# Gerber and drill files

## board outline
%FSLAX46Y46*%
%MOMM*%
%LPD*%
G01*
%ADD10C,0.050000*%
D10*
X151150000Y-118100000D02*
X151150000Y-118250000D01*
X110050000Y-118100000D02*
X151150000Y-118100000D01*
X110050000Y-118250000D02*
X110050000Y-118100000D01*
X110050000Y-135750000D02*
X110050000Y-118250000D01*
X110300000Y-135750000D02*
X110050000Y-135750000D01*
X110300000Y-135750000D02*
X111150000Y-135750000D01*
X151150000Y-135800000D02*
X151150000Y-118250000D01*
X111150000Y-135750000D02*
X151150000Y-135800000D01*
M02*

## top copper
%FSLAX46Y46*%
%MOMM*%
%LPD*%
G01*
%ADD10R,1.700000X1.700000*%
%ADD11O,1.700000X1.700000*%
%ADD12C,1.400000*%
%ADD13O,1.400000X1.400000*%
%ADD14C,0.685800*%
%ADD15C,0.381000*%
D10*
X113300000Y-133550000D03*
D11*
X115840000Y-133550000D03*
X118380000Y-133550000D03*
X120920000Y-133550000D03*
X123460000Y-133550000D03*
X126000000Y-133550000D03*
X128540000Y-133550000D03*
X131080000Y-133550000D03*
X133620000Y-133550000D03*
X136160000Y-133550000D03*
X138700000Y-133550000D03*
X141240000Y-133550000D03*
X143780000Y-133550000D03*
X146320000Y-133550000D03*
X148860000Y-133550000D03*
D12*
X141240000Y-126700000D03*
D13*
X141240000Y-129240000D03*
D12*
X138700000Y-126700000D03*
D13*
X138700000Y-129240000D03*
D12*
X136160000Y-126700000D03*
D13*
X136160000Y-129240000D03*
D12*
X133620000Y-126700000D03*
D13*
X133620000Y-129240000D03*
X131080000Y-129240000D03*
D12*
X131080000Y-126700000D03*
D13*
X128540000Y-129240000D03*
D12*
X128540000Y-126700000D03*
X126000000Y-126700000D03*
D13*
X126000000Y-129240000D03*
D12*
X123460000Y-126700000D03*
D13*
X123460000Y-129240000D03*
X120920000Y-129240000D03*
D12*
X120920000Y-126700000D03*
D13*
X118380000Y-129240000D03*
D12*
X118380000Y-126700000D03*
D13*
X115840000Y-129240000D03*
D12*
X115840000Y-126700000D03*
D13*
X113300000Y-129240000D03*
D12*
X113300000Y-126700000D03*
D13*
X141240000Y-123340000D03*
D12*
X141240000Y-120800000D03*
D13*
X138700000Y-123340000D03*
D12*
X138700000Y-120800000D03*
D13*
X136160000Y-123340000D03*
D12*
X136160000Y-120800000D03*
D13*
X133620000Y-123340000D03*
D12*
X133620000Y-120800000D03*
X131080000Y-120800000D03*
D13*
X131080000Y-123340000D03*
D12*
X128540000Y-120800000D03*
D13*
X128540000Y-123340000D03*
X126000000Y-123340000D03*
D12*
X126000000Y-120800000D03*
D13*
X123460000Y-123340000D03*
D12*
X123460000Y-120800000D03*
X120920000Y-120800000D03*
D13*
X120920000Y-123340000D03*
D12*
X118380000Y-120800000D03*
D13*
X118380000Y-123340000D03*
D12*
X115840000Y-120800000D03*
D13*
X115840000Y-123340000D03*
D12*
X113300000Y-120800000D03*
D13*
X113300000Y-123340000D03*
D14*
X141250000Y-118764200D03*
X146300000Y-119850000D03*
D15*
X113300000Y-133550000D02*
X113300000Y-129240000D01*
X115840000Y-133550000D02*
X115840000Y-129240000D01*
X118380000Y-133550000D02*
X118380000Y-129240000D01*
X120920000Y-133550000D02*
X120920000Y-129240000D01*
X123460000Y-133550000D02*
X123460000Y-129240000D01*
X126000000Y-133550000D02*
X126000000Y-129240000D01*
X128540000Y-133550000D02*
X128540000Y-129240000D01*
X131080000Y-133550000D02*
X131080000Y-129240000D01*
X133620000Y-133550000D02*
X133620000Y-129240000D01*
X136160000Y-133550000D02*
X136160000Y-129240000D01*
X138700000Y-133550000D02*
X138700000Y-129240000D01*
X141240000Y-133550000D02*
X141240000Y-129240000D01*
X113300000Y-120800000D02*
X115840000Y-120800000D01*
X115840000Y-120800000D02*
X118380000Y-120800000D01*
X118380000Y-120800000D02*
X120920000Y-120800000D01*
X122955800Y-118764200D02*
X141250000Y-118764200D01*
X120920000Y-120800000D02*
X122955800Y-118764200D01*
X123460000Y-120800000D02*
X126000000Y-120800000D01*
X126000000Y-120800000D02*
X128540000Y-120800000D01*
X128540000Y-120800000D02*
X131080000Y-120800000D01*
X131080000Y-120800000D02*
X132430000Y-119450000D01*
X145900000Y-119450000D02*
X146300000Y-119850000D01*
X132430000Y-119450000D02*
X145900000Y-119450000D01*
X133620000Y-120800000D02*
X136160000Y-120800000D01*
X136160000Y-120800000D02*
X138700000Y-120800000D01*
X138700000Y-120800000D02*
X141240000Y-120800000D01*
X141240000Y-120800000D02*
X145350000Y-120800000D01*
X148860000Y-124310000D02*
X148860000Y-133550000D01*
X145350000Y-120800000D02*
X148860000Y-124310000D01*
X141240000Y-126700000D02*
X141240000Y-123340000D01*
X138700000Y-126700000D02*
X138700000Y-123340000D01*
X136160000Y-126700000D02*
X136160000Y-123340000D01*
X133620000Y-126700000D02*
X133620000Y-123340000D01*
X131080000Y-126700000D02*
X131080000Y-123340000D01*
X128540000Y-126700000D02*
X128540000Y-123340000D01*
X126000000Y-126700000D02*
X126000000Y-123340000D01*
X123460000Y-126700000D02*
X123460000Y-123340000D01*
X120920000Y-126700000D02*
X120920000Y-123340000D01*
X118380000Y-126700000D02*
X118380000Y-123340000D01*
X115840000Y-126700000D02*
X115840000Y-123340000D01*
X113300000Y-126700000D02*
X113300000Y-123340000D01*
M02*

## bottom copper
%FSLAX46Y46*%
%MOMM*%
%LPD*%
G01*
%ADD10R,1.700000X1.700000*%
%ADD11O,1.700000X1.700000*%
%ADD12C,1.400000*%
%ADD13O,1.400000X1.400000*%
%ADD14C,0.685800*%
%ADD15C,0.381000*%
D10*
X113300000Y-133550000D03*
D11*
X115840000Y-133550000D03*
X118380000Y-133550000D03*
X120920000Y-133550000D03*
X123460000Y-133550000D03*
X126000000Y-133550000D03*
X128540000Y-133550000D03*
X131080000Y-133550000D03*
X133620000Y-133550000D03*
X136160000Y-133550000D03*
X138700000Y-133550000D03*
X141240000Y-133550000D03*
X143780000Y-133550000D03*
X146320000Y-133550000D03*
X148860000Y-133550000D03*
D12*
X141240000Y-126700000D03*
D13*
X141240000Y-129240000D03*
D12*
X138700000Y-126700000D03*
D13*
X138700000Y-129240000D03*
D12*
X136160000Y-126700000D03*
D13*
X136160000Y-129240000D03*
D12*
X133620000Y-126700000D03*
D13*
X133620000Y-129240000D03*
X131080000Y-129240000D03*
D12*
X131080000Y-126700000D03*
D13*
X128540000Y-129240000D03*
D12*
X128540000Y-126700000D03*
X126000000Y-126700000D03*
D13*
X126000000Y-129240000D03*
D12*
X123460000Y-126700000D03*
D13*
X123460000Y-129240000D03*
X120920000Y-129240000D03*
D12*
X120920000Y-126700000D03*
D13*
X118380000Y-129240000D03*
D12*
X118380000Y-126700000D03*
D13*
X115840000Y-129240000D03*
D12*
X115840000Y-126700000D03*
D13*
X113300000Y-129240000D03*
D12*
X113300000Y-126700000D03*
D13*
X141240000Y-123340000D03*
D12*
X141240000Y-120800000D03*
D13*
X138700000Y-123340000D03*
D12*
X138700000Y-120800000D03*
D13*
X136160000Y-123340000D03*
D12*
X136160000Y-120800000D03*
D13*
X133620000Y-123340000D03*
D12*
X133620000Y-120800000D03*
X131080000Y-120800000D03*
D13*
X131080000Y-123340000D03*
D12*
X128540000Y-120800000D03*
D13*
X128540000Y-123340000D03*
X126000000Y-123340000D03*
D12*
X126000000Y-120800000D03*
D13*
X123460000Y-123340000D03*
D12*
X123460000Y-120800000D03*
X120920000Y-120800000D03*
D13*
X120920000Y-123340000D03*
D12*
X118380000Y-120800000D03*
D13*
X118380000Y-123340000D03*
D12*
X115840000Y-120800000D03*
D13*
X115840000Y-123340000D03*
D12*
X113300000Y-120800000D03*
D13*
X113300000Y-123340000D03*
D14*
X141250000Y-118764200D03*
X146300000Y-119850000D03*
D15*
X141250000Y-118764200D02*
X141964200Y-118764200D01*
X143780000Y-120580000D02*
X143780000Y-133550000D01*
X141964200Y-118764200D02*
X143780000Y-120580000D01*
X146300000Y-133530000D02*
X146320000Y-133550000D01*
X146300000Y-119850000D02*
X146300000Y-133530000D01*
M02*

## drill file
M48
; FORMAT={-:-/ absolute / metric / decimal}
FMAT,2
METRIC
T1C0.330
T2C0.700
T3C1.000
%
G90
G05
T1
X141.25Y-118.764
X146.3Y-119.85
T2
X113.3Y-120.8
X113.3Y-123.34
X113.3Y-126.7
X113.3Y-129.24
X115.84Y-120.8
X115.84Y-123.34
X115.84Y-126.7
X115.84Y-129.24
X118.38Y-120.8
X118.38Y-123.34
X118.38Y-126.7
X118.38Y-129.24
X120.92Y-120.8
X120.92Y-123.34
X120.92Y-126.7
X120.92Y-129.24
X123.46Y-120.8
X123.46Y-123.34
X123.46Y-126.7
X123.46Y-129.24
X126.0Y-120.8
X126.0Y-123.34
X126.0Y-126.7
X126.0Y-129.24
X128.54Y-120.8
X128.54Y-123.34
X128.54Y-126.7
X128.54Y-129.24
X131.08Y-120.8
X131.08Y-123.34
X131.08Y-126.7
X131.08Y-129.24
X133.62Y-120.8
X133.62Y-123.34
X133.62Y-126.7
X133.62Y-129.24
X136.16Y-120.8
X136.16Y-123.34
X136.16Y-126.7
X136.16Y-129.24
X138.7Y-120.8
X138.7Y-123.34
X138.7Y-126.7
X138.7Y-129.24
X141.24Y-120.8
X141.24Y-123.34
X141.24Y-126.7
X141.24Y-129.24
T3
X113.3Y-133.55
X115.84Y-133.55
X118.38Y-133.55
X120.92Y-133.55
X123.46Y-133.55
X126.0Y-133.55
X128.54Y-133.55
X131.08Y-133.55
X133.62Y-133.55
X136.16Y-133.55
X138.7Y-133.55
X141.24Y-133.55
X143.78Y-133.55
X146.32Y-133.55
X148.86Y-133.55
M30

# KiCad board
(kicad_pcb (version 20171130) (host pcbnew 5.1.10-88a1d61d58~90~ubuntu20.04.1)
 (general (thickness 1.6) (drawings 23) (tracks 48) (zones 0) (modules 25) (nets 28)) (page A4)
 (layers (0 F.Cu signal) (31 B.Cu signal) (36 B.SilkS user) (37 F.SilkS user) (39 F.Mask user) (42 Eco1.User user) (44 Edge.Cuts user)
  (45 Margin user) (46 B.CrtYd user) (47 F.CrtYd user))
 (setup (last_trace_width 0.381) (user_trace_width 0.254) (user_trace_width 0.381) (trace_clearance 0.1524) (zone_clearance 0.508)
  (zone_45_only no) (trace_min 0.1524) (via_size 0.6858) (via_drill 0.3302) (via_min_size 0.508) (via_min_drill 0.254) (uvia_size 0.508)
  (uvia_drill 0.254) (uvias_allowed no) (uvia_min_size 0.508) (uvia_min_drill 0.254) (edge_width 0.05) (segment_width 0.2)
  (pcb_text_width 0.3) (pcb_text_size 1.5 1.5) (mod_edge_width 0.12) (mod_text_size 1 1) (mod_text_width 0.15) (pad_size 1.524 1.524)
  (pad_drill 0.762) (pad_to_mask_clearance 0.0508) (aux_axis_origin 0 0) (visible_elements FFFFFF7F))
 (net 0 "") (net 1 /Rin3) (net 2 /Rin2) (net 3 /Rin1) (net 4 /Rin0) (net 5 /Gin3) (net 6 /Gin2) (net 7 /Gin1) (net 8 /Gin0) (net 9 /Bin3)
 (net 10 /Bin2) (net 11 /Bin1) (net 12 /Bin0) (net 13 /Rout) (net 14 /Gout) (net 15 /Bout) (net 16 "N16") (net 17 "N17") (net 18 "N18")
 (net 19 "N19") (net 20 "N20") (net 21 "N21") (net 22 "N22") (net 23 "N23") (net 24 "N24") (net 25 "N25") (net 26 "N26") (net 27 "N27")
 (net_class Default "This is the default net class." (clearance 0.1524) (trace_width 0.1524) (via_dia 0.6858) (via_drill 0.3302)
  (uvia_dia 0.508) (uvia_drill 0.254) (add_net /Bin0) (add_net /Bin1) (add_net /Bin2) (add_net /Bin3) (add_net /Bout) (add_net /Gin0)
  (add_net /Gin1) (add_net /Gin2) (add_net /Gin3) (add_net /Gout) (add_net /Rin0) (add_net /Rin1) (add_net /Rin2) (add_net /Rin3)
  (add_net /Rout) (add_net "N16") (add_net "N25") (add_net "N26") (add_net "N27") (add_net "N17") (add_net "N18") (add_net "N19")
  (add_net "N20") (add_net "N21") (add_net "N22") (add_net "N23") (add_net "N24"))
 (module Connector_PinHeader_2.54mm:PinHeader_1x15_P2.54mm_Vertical (layer F.Cu) (at 113.3 133.55 90)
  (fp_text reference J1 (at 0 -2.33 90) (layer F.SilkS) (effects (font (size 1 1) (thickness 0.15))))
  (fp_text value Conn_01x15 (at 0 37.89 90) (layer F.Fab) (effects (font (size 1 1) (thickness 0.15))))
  (pad 1 thru_hole rect (at 0 0 90) (size 1.7 1.7) (drill 1) (layers *.Cu *.Mask) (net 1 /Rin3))
  (pad 2 thru_hole oval (at 0 2.54 90) (size 1.7 1.7) (drill 1) (layers *.Cu *.Mask) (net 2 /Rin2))
  (pad 3 thru_hole oval (at 0 5.08 90) (size 1.7 1.7) (drill 1) (layers *.Cu *.Mask) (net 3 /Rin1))
  (pad 4 thru_hole oval (at 0 7.62 90) (size 1.7 1.7) (drill 1) (layers *.Cu *.Mask) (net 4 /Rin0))
  (pad 5 thru_hole oval (at 0 10.16 90) (size 1.7 1.7) (drill 1) (layers *.Cu *.Mask) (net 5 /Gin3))
  (pad 6 thru_hole oval (at 0 12.7 90) (size 1.7 1.7) (drill 1) (layers *.Cu *.Mask) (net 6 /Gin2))
  (pad 7 thru_hole oval (at 0 15.24 90) (size 1.7 1.7) (drill 1) (layers *.Cu *.Mask) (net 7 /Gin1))
  (pad 8 thru_hole oval (at 0 17.78 90) (size 1.7 1.7) (drill 1) (layers *.Cu *.Mask) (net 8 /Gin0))
  (pad 9 thru_hole oval (at 0 20.32 90) (size 1.7 1.7) (drill 1) (layers *.Cu *.Mask) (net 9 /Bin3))
  (pad 10 thru_hole oval (at 0 22.86 90) (size 1.7 1.7) (drill 1) (layers *.Cu *.Mask) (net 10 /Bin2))
  (pad 11 thru_hole oval (at 0 25.4 90) (size 1.7 1.7) (drill 1) (layers *.Cu *.Mask) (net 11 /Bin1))
  (pad 12 thru_hole oval (at 0 27.94 90) (size 1.7 1.7) (drill 1) (layers *.Cu *.Mask) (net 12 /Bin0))
  (pad 13 thru_hole oval (at 0 30.48 90) (size 1.7 1.7) (drill 1) (layers *.Cu *.Mask) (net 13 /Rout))
  (pad 14 thru_hole oval (at 0 33.02 90) (size 1.7 1.7) (drill 1) (layers *.Cu *.Mask) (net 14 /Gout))
  (pad 15 thru_hole oval (at 0 35.56 90) (size 1.7 1.7) (drill 1) (layers *.Cu *.Mask) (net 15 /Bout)))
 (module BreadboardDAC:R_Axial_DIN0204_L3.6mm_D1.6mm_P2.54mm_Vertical (layer F.Cu) (at 141.24 126.7 270)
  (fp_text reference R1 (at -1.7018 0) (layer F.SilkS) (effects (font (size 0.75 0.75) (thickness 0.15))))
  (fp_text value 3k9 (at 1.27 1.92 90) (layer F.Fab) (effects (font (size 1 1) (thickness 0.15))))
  (pad 1 thru_hole circle (at 0 0 270) (size 1.4 1.4) (drill 0.7) (layers *.Cu *.Mask) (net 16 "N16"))
  (pad 2 thru_hole oval (at 2.54 0 270) (size 1.4 1.4) (drill 0.7) (layers *.Cu *.Mask) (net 12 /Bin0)))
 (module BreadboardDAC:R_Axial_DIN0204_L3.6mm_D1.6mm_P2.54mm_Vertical (layer F.Cu) (at 138.7 126.7 270)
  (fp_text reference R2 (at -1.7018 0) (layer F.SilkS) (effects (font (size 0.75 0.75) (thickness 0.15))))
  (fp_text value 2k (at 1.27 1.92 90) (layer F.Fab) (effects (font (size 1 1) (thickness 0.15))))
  (pad 1 thru_hole circle (at 0 0 270) (size 1.4 1.4) (drill 0.7) (layers *.Cu *.Mask) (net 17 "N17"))
  (pad 2 thru_hole oval (at 2.54 0 270) (size 1.4 1.4) (drill 0.7) (layers *.Cu *.Mask) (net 11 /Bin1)))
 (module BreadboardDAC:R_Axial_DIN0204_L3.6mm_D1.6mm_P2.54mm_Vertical (layer F.Cu) (at 136.16 126.7 270)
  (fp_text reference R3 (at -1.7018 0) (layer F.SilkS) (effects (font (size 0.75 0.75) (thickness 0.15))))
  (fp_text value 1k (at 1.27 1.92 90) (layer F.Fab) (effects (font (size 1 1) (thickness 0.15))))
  (pad 1 thru_hole circle (at 0 0 270) (size 1.4 1.4) (drill 0.7) (layers *.Cu *.Mask) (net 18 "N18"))
  (pad 2 thru_hole oval (at 2.54 0 270) (size 1.4 1.4) (drill 0.7) (layers *.Cu *.Mask) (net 10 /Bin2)))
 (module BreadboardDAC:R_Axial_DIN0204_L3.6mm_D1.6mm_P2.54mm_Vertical (layer F.Cu) (at 133.62 126.7 270)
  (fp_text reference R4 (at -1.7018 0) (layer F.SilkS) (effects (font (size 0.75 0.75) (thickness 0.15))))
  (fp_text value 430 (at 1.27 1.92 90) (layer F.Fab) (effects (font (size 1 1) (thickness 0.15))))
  (pad 1 thru_hole circle (at 0 0 270) (size 1.4 1.4) (drill 0.7) (layers *.Cu *.Mask) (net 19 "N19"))
  (pad 2 thru_hole oval (at 2.54 0 270) (size 1.4 1.4) (drill 0.7) (layers *.Cu *.Mask) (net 9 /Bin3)))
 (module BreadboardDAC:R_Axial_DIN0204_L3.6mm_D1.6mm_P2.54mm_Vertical (layer F.Cu) (at 131.08 126.7 270)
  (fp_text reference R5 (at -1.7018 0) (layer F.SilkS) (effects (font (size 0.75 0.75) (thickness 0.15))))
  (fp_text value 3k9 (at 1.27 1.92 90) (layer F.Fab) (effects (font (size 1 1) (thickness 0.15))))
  (pad 2 thru_hole oval (at 2.54 0 270) (size 1.4 1.4) (drill 0.7) (layers *.Cu *.Mask) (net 8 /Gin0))
  (pad 1 thru_hole circle (at 0 0 270) (size 1.4 1.4) (drill 0.7) (layers *.Cu *.Mask) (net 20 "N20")))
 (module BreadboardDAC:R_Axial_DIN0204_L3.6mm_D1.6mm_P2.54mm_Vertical (layer F.Cu) (at 128.54 126.7 270)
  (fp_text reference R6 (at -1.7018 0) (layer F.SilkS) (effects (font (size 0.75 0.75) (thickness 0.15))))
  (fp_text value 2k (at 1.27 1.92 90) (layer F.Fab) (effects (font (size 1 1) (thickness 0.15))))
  (pad 2 thru_hole oval (at 2.54 0 270) (size 1.4 1.4) (drill 0.7) (layers *.Cu *.Mask) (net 7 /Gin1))
  (pad 1 thru_hole circle (at 0 0 270) (size 1.4 1.4) (drill 0.7) (layers *.Cu *.Mask) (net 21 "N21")))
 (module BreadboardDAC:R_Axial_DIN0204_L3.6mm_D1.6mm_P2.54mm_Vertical (layer F.Cu) (at 126 126.7 270)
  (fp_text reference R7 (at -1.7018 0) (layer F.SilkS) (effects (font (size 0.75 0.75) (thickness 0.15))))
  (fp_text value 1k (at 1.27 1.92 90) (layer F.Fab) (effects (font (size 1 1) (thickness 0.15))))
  (pad 1 thru_hole circle (at 0 0 270) (size 1.4 1.4) (drill 0.7) (layers *.Cu *.Mask) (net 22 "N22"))
  (pad 2 thru_hole oval (at 2.54 0 270) (size 1.4 1.4) (drill 0.7) (layers *.Cu *.Mask) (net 6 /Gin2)))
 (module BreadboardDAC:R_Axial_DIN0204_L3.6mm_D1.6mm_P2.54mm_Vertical (layer F.Cu) (at 123.46 126.7 270)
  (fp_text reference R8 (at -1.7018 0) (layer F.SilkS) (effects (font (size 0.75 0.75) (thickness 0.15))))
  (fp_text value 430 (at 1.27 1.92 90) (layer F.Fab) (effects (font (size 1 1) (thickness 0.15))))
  (pad 1 thru_hole circle (at 0 0 270) (size 1.4 1.4) (drill 0.7) (layers *.Cu *.Mask) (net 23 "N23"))
  (pad 2 thru_hole oval (at 2.54 0 270) (size 1.4 1.4) (drill 0.7) (layers *.Cu *.Mask) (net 5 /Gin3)))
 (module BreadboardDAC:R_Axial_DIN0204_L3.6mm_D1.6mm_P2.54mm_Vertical (layer F.Cu) (at 120.92 126.7 270)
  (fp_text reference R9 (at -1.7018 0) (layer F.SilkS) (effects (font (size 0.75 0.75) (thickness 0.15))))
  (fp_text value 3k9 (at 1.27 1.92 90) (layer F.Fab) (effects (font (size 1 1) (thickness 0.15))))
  (pad 2 thru_hole oval (at 2.54 0 270) (size 1.4 1.4) (drill 0.7) (layers *.Cu *.Mask) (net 4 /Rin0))
  (pad 1 thru_hole circle (at 0 0 270) (size 1.4 1.4) (drill 0.7) (layers *.Cu *.Mask) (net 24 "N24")))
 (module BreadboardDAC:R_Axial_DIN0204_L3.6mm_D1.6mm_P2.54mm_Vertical (layer F.Cu) (at 118.38 126.7 270)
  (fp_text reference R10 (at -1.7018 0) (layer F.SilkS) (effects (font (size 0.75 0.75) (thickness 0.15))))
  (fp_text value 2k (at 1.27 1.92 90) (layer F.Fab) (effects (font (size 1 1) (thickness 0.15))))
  (pad 2 thru_hole oval (at 2.54 0 270) (size 1.4 1.4) (drill 0.7) (layers *.Cu *.Mask) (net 3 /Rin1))
  (pad 1 thru_hole circle (at 0 0 270) (size 1.4 1.4) (drill 0.7) (layers *.Cu *.Mask) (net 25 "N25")))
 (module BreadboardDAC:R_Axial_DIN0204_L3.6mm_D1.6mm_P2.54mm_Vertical (layer F.Cu) (at 115.84 126.7 270)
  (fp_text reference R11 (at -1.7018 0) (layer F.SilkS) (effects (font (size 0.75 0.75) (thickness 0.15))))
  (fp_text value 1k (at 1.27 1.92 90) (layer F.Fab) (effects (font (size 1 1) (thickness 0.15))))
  (pad 2 thru_hole oval (at 2.54 0 270) (size 1.4 1.4) (drill 0.7) (layers *.Cu *.Mask) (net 2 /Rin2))
  (pad 1 thru_hole circle (at 0 0 270) (size 1.4 1.4) (drill 0.7) (layers *.Cu *.Mask) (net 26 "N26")))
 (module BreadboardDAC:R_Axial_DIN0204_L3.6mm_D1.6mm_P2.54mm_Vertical (layer F.Cu) (at 113.3 126.7 270)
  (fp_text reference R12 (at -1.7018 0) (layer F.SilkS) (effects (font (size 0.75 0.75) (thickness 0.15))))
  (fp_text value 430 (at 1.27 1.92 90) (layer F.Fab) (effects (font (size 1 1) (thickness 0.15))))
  (pad 2 thru_hole oval (at 2.54 0 270) (size 1.4 1.4) (drill 0.7) (layers *.Cu *.Mask) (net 1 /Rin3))
  (pad 1 thru_hole circle (at 0 0 270) (size 1.4 1.4) (drill 0.7) (layers *.Cu *.Mask) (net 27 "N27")))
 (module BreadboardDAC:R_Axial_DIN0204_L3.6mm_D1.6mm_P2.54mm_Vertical (layer F.Cu) (at 141.24 120.8 270)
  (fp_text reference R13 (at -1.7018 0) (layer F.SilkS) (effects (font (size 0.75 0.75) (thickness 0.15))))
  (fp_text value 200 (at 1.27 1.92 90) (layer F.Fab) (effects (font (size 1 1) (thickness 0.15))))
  (pad 2 thru_hole oval (at 2.54 0 270) (size 1.4 1.4) (drill 0.7) (layers *.Cu *.Mask) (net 16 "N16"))
  (pad 1 thru_hole circle (at 0 0 270) (size 1.4 1.4) (drill 0.7) (layers *.Cu *.Mask) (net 15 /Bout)))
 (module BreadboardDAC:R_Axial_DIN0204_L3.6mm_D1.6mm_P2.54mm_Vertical (layer F.Cu) (at 138.7 120.8 270)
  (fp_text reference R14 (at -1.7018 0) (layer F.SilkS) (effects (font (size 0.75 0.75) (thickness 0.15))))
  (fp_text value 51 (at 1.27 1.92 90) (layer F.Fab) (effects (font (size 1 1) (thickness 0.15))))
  (pad 2 thru_hole oval (at 2.54 0 270) (size 1.4 1.4) (drill 0.7) (layers *.Cu *.Mask) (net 17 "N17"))
  (pad 1 thru_hole circle (at 0 0 270) (size 1.4 1.4) (drill 0.7) (layers *.Cu *.Mask) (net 15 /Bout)))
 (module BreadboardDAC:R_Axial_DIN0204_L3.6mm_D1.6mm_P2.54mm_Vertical (layer F.Cu) (at 136.16 120.8 270)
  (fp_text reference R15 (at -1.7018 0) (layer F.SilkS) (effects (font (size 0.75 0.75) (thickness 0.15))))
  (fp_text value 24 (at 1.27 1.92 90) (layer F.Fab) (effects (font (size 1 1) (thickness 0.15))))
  (pad 2 thru_hole oval (at 2.54 0 270) (size 1.4 1.4) (drill 0.7) (layers *.Cu *.Mask) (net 18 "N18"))
  (pad 1 thru_hole circle (at 0 0 270) (size 1.4 1.4) (drill 0.7) (layers *.Cu *.Mask) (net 15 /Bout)))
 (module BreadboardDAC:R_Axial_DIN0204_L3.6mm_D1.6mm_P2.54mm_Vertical (layer F.Cu) (at 133.62 120.8 270)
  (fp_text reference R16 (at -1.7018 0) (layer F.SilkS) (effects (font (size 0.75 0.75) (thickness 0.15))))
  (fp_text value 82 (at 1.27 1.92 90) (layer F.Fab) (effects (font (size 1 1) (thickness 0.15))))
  (pad 2 thru_hole oval (at 2.54 0 270) (size 1.4 1.4) (drill 0.7) (layers *.Cu *.Mask) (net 19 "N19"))
  (pad 1 thru_hole circle (at 0 0 270) (size 1.4 1.4) (drill 0.7) (layers *.Cu *.Mask) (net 15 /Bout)))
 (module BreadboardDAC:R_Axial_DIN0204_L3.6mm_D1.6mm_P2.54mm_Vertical (layer F.Cu) (at 131.08 120.8 270)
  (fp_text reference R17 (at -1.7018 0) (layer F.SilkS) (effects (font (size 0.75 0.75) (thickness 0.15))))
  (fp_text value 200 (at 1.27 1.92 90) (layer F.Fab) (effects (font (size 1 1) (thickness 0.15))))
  (pad 1 thru_hole circle (at 0 0 270) (size 1.4 1.4) (drill 0.7) (layers *.Cu *.Mask) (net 14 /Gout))
  (pad 2 thru_hole oval (at 2.54 0 270) (size 1.4 1.4) (drill 0.7) (layers *.Cu *.Mask) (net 20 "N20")))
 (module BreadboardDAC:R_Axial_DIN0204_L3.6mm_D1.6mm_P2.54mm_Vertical (layer F.Cu) (at 128.54 120.8 270)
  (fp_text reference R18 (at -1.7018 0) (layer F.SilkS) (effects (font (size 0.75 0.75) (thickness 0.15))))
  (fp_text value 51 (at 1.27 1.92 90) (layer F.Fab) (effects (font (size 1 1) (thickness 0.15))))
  (pad 1 thru_hole circle (at 0 0 270) (size 1.4 1.4) (drill 0.7) (layers *.Cu *.Mask) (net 14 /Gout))
  (pad 2 thru_hole oval (at 2.54 0 270) (size 1.4 1.4) (drill 0.7) (layers *.Cu *.Mask) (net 21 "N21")))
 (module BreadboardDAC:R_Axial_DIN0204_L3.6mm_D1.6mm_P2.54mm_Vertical (layer F.Cu) (at 126 120.8 270)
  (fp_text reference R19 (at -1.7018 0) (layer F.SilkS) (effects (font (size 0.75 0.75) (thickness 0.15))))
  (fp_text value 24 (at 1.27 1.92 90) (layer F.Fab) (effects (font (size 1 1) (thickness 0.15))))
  (pad 2 thru_hole oval (at 2.54 0 270) (size 1.4 1.4) (drill 0.7) (layers *.Cu *.Mask) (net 22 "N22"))
  (pad 1 thru_hole circle (at 0 0 270) (size 1.4 1.4) (drill 0.7) (layers *.Cu *.Mask) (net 14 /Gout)))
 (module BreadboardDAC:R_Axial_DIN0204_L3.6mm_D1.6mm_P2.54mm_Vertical (layer F.Cu) (at 123.46 120.8 270)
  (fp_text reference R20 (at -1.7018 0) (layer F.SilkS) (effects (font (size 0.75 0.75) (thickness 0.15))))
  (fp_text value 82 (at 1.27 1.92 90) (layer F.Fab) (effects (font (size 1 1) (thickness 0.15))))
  (pad 2 thru_hole oval (at 2.54 0 270) (size 1.4 1.4) (drill 0.7) (layers *.Cu *.Mask) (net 23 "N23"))
  (pad 1 thru_hole circle (at 0 0 270) (size 1.4 1.4) (drill 0.7) (layers *.Cu *.Mask) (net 14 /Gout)))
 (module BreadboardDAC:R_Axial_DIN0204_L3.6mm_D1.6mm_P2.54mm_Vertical (layer F.Cu) (at 120.92 120.8 270)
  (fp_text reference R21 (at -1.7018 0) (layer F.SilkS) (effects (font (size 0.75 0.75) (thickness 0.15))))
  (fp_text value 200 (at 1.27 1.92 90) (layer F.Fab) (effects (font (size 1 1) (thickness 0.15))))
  (pad 1 thru_hole circle (at 0 0 270) (size 1.4 1.4) (drill 0.7) (layers *.Cu *.Mask) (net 13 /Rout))
  (pad 2 thru_hole oval (at 2.54 0 270) (size 1.4 1.4) (drill 0.7) (layers *.Cu *.Mask) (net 24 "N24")))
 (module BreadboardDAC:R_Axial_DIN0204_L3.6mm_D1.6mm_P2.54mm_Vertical (layer F.Cu) (at 118.38 120.8 270)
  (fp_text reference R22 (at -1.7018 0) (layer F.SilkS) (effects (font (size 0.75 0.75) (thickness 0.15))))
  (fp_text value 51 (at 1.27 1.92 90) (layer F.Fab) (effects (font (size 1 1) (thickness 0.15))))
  (pad 1 thru_hole circle (at 0 0 270) (size 1.4 1.4) (drill 0.7) (layers *.Cu *.Mask) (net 13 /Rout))
  (pad 2 thru_hole oval (at 2.54 0 270) (size 1.4 1.4) (drill 0.7) (layers *.Cu *.Mask) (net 25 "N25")))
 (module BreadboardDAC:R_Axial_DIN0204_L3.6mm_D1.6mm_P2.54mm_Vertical (layer F.Cu) (at 115.84 120.8 270)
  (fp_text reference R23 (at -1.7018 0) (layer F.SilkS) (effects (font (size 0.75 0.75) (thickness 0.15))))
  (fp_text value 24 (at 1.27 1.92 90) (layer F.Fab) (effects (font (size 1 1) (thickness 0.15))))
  (pad 1 thru_hole circle (at 0 0 270) (size 1.4 1.4) (drill 0.7) (layers *.Cu *.Mask) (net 13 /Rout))
  (pad 2 thru_hole oval (at 2.54 0 270) (size 1.4 1.4) (drill 0.7) (layers *.Cu *.Mask) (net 26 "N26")))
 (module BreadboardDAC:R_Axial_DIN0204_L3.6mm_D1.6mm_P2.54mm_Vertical (layer F.Cu) (at 113.3 120.8 270)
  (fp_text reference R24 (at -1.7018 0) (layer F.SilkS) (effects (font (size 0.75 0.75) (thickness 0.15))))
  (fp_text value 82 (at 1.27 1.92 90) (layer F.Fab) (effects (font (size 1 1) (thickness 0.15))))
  (pad 1 thru_hole circle (at 0 0 270) (size 1.4 1.4) (drill 0.7) (layers *.Cu *.Mask) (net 13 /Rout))
  (pad 2 thru_hole oval (at 2.54 0 270) (size 1.4 1.4) (drill 0.7) (layers *.Cu *.Mask) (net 27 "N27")))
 (gr_line (start 151.15 118.1) (end 151.15 118.25) (layer Edge.Cuts) (width 0.05))
 (gr_line (start 110.05 118.1) (end 151.15 118.1) (layer Edge.Cuts) (width 0.05))
 (gr_line (start 110.05 118.25) (end 110.05 118.1) (layer Edge.Cuts) (width 0.05))
 (gr_line (start 110.05 135.75) (end 110.05 118.25) (layer Edge.Cuts) (width 0.05))
 (gr_line (start 110.3 135.75) (end 110.05 135.75) (layer Edge.Cuts) (width 0.05))
 (gr_line (start 110.3 135.75) (end 111.15 135.75) (layer Edge.Cuts) (width 0.05))
 (gr_line (start 151.15 135.8) (end 151.15 118.25) (layer Edge.Cuts) (width 0.05))
 (gr_line (start 111.15 135.75) (end 151.15 135.8) (layer Edge.Cuts) (width 0.05))
 (segment (start 113.3 133.55) (end 113.3 129.24) (width 0.381) (layer F.Cu) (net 1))
 (segment (start 115.84 133.55) (end 115.84 129.24) (width 0.381) (layer F.Cu) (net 2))
 (segment (start 118.38 133.55) (end 118.38 129.24) (width 0.381) (layer F.Cu) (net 3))
 (segment (start 120.92 133.55) (end 120.92 129.24) (width 0.381) (layer F.Cu) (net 4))
 (segment (start 123.46 133.55) (end 123.46 129.24) (width 0.381) (layer F.Cu) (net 5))
 (segment (start 126 133.55) (end 126 129.24) (width 0.381) (layer F.Cu) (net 6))
 (segment (start 128.54 133.55) (end 128.54 129.24) (width 0.381) (layer F.Cu) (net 7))
 (segment (start 131.08 133.55) (end 131.08 129.24) (width 0.381) (layer F.Cu) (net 8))
 (segment (start 133.62 133.55) (end 133.62 129.24) (width 0.381) (layer F.Cu) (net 9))
 (segment (start 136.16 133.55) (end 136.16 129.24) (width 0.381) (layer F.Cu) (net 10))
 (segment (start 138.7 133.55) (end 138.7 129.24) (width 0.381) (layer F.Cu) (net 11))
 (segment (start 141.24 133.55) (end 141.24 129.24) (width 0.381) (layer F.Cu) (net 12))
 (segment (start 113.3 120.8) (end 115.84 120.8) (width 0.381) (layer F.Cu) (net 13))
 (segment (start 115.84 120.8) (end 118.38 120.8) (width 0.381) (layer F.Cu) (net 13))
 (segment (start 118.38 120.8) (end 120.92 120.8) (width 0.381) (layer F.Cu) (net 13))
 (segment (start 122.9558 118.7642) (end 141.25 118.7642) (width 0.381) (layer F.Cu) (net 13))
 (via (at 141.25 118.7642) (size 0.6858) (drill 0.3302) (layers F.Cu B.Cu) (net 13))
 (segment (start 120.92 120.8) (end 122.9558 118.7642) (width 0.381) (layer F.Cu) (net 13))
 (segment (start 141.25 118.7642) (end 141.9642 118.7642) (width 0.381) (layer B.Cu) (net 13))
 (segment (start 143.78 120.58) (end 143.78 133.55) (width 0.381) (layer B.Cu) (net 13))
 (segment (start 141.9642 118.7642) (end 143.78 120.58) (width 0.381) (layer B.Cu) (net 13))
 (segment (start 123.46 120.8) (end 126 120.8) (width 0.381) (layer F.Cu) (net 14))
 (segment (start 126 120.8) (end 128.54 120.8) (width 0.381) (layer F.Cu) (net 14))
 (segment (start 128.54 120.8) (end 131.08 120.8) (width 0.381) (layer F.Cu) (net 14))
 (segment (start 131.08 120.8) (end 132.43 119.45) (width 0.381) (layer F.Cu) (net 14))
 (via (at 146.3 119.85) (size 0.6858) (drill 0.3302) (layers F.Cu B.Cu) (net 14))
 (segment (start 145.9 119.45) (end 146.3 119.85) (width 0.381) (layer F.Cu) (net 14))
 (segment (start 132.43 119.45) (end 145.9 119.45) (width 0.381) (layer F.Cu) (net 14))
 (segment (start 146.3 133.53) (end 146.32 133.55) (width 0.381) (layer B.Cu) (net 14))
 (segment (start 146.3 119.85) (end 146.3 133.53) (width 0.381) (layer B.Cu) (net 14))
 (segment (start 133.62 120.8) (end 136.16 120.8) (width 0.381) (layer F.Cu) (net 15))
 (segment (start 136.16 120.8) (end 138.7 120.8) (width 0.381) (layer F.Cu) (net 15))
 (segment (start 138.7 120.8) (end 141.24 120.8) (width 0.381) (layer F.Cu) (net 15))
 (segment (start 141.24 120.8) (end 145.35 120.8) (width 0.381) (layer F.Cu) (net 15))
 (segment (start 148.86 124.31) (end 148.86 133.55) (width 0.381) (layer F.Cu) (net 15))
 (segment (start 145.35 120.8) (end 148.86 124.31) (width 0.381) (layer F.Cu) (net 15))
 (segment (start 141.24 126.7) (end 141.24 123.34) (width 0.381) (layer F.Cu) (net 16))
 (segment (start 138.7 126.7) (end 138.7 123.34) (width 0.381) (layer F.Cu) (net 17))
 (segment (start 136.16 126.7) (end 136.16 123.34) (width 0.381) (layer F.Cu) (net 18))
 (segment (start 133.62 126.7) (end 133.62 123.34) (width 0.381) (layer F.Cu) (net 19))
 (segment (start 131.08 126.7) (end 131.08 123.34) (width 0.381) (layer F.Cu) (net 20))
 (segment (start 128.54 126.7) (end 128.54 123.34) (width 0.381) (layer F.Cu) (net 21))
 (segment (start 126 126.7) (end 126 123.34) (width 0.381) (layer F.Cu) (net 22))
 (segment (start 123.46 126.7) (end 123.46 123.34) (width 0.381) (layer F.Cu) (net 23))
 (segment (start 120.92 126.7) (end 120.92 123.34) (width 0.381) (layer F.Cu) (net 24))
 (segment (start 118.38 126.7) (end 118.38 123.34) (width 0.381) (layer F.Cu) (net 25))
 (segment (start 115.84 126.7) (end 115.84 123.34) (width 0.381) (layer F.Cu) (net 26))
 (segment (start 113.3 126.7) (end 113.3 123.34) (width 0.381) (layer F.Cu) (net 27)))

